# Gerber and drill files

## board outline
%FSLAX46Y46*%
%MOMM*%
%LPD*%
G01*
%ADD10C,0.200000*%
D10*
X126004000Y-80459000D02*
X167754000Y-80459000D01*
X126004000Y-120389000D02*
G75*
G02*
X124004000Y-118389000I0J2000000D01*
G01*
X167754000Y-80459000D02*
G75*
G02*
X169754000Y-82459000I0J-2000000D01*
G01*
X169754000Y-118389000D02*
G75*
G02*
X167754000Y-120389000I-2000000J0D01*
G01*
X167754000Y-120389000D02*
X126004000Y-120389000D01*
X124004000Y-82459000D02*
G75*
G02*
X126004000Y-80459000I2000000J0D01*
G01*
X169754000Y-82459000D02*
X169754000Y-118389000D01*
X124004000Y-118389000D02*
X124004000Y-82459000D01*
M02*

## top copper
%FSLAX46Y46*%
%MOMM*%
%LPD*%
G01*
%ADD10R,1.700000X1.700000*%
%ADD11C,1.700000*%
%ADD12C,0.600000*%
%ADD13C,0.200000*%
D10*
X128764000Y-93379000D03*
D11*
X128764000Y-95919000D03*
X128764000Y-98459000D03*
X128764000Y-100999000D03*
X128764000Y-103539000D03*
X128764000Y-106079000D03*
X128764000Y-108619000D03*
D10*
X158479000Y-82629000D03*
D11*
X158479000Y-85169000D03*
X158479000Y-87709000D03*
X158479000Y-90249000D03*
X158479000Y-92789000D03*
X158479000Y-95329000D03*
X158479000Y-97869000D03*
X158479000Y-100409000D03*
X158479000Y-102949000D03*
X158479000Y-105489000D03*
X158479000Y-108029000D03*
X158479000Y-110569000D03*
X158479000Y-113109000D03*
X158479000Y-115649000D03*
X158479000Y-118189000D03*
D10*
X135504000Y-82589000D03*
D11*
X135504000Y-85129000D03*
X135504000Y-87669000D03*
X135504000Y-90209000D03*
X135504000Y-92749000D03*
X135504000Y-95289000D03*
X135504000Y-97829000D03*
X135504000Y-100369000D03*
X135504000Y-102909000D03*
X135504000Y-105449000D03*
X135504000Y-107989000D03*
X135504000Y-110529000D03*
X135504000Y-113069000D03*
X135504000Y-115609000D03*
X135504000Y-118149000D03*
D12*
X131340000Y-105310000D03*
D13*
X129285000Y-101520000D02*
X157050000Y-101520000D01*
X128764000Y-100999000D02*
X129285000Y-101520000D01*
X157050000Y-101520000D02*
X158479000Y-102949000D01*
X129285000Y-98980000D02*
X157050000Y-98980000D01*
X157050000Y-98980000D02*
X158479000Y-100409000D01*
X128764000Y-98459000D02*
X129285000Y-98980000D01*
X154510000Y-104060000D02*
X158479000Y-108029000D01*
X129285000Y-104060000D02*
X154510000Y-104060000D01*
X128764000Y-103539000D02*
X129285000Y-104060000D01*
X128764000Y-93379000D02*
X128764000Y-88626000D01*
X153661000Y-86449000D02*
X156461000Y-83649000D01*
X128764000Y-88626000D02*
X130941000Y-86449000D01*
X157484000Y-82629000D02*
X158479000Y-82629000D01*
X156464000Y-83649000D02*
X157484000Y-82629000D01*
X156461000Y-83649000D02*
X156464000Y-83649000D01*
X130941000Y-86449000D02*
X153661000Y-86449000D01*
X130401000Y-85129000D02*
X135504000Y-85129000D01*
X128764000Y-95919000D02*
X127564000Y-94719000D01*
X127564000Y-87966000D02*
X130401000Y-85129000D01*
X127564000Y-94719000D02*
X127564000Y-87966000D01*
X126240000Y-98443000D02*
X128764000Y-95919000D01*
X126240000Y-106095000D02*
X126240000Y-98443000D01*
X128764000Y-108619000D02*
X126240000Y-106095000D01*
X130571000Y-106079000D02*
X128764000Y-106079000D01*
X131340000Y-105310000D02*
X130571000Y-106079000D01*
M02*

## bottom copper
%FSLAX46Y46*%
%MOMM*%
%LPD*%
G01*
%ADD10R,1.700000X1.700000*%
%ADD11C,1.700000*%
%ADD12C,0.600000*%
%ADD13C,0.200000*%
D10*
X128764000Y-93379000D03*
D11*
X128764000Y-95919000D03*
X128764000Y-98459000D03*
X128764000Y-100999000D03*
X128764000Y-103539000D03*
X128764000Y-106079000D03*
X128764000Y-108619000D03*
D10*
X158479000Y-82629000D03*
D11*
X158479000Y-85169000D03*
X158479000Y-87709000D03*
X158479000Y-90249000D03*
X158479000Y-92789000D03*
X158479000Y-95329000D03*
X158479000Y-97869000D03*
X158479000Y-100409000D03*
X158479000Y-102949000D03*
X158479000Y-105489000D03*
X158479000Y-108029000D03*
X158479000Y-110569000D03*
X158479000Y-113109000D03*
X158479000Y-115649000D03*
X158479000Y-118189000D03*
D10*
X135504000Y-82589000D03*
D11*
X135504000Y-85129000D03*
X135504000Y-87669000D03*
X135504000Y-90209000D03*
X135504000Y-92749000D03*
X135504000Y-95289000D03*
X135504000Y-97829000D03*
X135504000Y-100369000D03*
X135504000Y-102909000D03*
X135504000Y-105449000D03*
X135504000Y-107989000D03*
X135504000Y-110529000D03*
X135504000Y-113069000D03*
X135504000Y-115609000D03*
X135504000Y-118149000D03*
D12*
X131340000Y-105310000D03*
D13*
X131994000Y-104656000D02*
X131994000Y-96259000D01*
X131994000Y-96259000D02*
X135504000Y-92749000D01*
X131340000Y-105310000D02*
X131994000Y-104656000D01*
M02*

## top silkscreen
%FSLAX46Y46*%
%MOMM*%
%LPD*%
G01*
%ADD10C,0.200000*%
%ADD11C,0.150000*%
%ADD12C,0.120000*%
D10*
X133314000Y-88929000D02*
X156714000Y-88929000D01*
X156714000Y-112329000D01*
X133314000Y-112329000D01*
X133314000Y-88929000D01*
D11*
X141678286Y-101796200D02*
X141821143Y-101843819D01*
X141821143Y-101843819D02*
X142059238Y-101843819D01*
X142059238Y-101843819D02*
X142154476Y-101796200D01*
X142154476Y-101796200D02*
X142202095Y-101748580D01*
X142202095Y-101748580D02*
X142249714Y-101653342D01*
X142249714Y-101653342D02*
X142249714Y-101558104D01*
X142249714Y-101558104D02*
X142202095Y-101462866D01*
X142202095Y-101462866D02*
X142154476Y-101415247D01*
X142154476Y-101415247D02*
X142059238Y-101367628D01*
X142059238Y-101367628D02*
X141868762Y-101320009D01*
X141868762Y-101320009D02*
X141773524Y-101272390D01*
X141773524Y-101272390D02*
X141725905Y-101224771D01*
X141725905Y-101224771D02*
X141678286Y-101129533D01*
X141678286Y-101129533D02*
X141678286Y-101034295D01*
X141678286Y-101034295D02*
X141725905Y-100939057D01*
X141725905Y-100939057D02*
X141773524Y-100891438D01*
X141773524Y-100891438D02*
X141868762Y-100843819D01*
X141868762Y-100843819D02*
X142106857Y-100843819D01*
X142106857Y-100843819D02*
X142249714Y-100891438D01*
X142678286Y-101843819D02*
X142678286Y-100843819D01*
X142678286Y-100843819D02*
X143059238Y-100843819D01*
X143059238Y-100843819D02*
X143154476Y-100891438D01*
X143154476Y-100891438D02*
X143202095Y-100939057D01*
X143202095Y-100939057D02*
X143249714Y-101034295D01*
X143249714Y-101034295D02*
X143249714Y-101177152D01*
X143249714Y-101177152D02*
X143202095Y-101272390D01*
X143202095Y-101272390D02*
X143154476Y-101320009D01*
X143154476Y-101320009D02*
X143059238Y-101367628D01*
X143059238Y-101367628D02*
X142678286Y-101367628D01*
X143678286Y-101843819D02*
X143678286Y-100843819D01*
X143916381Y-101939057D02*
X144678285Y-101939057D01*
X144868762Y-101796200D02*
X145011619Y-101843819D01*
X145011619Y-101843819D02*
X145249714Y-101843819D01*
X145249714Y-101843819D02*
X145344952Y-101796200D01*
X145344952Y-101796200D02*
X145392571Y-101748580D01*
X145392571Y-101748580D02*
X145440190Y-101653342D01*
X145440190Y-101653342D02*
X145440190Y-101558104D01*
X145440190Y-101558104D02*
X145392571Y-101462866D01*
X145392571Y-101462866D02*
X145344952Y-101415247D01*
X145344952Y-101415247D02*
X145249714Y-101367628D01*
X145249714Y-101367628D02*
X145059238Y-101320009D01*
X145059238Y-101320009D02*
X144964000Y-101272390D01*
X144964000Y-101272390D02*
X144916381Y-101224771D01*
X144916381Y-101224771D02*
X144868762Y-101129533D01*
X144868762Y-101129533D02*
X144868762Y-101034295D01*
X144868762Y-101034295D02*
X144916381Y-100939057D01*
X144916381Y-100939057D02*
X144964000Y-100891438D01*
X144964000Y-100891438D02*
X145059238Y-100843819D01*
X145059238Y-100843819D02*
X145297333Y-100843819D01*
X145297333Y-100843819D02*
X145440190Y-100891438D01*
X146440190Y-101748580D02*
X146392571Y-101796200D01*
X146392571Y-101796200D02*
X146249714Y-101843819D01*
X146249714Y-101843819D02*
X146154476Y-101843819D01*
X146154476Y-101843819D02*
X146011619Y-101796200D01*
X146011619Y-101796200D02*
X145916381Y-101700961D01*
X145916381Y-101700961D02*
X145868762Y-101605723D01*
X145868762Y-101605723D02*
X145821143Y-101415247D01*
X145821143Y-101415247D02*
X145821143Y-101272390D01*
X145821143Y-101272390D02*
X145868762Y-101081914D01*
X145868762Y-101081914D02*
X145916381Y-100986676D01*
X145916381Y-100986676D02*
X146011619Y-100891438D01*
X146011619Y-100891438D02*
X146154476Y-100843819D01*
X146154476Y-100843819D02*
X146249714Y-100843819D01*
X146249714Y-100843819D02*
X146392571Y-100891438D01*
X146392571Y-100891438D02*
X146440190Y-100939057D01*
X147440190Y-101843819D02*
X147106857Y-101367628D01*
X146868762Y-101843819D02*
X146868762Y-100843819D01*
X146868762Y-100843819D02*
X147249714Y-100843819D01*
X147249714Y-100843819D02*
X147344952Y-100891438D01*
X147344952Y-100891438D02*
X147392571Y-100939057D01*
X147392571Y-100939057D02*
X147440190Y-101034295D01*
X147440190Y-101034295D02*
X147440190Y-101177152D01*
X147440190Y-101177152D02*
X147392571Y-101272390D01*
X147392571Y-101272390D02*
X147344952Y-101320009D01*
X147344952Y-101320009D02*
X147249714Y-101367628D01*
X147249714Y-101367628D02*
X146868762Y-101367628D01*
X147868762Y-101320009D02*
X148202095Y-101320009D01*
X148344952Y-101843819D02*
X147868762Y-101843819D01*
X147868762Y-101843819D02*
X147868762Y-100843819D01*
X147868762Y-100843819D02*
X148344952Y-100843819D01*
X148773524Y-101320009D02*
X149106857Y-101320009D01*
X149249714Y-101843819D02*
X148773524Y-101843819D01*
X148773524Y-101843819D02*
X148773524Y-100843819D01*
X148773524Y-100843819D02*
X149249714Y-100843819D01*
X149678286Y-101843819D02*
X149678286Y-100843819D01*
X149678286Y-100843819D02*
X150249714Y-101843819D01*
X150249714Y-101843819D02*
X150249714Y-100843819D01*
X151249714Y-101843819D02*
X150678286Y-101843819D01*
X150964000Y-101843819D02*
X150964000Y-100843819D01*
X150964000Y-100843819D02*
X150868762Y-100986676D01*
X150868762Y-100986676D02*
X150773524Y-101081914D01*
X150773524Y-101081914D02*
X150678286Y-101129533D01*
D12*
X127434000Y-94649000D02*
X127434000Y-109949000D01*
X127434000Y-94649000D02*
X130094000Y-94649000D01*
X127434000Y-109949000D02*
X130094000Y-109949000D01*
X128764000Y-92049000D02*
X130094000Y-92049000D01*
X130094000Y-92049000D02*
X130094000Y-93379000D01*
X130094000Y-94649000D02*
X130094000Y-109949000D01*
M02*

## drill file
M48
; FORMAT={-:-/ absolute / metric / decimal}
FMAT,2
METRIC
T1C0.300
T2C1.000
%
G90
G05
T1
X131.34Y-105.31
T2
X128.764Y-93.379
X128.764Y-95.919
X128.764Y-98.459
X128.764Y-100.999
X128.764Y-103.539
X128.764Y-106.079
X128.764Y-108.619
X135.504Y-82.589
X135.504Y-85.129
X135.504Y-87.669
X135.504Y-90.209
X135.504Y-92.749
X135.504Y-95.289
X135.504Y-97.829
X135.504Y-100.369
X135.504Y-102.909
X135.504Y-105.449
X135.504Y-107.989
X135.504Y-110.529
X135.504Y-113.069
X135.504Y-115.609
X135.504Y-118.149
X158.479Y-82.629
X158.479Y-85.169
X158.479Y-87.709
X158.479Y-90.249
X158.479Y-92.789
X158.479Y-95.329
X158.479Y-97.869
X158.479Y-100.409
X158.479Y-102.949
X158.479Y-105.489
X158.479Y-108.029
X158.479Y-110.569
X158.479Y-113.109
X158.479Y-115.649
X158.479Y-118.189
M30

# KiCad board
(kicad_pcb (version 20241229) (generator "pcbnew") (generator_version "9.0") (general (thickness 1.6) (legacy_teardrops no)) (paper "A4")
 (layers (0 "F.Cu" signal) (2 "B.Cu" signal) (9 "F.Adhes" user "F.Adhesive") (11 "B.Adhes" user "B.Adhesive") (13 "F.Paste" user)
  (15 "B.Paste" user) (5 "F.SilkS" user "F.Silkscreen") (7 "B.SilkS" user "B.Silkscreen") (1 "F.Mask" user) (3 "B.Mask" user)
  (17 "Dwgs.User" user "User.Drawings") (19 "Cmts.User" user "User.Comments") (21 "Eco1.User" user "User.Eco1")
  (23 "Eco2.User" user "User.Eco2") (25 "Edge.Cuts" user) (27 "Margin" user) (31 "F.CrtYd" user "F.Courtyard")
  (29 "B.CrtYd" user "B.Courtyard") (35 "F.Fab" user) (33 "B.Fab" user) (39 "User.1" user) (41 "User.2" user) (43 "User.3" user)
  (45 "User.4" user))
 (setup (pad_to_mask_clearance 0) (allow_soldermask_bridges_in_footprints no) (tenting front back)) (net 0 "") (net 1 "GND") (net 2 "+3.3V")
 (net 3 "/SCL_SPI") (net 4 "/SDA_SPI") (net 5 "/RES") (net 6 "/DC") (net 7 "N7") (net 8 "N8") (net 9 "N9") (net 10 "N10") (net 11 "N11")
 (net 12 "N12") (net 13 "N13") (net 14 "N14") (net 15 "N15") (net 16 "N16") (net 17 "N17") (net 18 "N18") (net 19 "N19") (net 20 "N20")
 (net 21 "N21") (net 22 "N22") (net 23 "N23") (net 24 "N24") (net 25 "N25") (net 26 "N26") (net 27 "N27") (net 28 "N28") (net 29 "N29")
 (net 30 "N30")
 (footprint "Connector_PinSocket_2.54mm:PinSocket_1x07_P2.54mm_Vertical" (layer "F.Cu") (at 128.764 93.379)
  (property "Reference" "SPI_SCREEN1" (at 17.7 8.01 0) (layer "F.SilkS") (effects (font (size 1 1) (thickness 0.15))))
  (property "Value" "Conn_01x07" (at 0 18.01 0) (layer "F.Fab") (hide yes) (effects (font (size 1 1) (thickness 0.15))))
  (fp_line (start -1.33 1.27) (end -1.33 16.57) (stroke (width 0.12) (type solid)) (layer "F.SilkS"))
  (fp_line (start -1.33 1.27) (end 1.33 1.27) (stroke (width 0.12) (type solid)) (layer "F.SilkS"))
  (fp_line (start -1.33 16.57) (end 1.33 16.57) (stroke (width 0.12) (type solid)) (layer "F.SilkS"))
  (fp_line (start 0 -1.33) (end 1.33 -1.33) (stroke (width 0.12) (type solid)) (layer "F.SilkS"))
  (fp_line (start 1.33 -1.33) (end 1.33 0) (stroke (width 0.12) (type solid)) (layer "F.SilkS"))
  (fp_line (start 1.33 1.27) (end 1.33 16.57) (stroke (width 0.12) (type solid)) (layer "F.SilkS"))
  (pad "1" thru_hole rect (at 0 0) (size 1.7 1.7) (drill 1) (layers "*.Cu" "*.Mask") (remove_unused_layers no) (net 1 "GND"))
  (pad "2" thru_hole circle (at 0 2.54) (size 1.7 1.7) (drill 1) (layers "*.Cu" "*.Mask") (remove_unused_layers no) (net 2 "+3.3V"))
  (pad "3" thru_hole circle (at 0 5.08) (size 1.7 1.7) (drill 1) (layers "*.Cu" "*.Mask") (remove_unused_layers no) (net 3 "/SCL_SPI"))
  (pad "4" thru_hole circle (at 0 7.62) (size 1.7 1.7) (drill 1) (layers "*.Cu" "*.Mask") (remove_unused_layers no) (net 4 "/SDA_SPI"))
  (pad "5" thru_hole circle (at 0 10.16) (size 1.7 1.7) (drill 1) (layers "*.Cu" "*.Mask") (remove_unused_layers no) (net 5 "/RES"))
  (pad "6" thru_hole circle (at 0 12.7) (size 1.7 1.7) (drill 1) (layers "*.Cu" "*.Mask") (remove_unused_layers no) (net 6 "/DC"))
  (pad "7" thru_hole circle (at 0 15.24) (size 1.7 1.7) (drill 1) (layers "*.Cu" "*.Mask") (remove_unused_layers no) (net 2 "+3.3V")))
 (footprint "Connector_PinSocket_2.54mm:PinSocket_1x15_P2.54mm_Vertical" (layer "B.Cu") (at 158.479 82.629 180)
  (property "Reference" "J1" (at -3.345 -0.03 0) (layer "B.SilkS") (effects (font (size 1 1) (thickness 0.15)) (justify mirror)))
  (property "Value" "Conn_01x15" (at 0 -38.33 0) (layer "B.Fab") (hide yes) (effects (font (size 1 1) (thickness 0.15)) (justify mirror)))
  (pad "1" thru_hole rect (at 0 0 180) (size 1.7 1.7) (drill 1) (layers "*.Cu" "*.Mask") (remove_unused_layers no) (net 1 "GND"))
  (pad "2" thru_hole circle (at 0 -2.54 180) (size 1.7 1.7) (drill 1) (layers "*.Cu" "*.Mask") (remove_unused_layers no) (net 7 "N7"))
  (pad "3" thru_hole circle (at 0 -5.08 180) (size 1.7 1.7) (drill 1) (layers "*.Cu" "*.Mask") (remove_unused_layers no) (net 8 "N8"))
  (pad "4" thru_hole circle (at 0 -7.62 180) (size 1.7 1.7) (drill 1) (layers "*.Cu" "*.Mask") (remove_unused_layers no) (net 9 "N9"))
  (pad "5" thru_hole circle (at 0 -10.16 180) (size 1.7 1.7) (drill 1) (layers "*.Cu" "*.Mask") (remove_unused_layers no) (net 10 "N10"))
  (pad "6" thru_hole circle (at 0 -12.7 180) (size 1.7 1.7) (drill 1) (layers "*.Cu" "*.Mask") (remove_unused_layers no) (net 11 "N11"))
  (pad "7" thru_hole circle (at 0 -15.24 180) (size 1.7 1.7) (drill 1) (layers "*.Cu" "*.Mask") (remove_unused_layers no) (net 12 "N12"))
  (pad "8" thru_hole circle (at 0 -17.78 180) (size 1.7 1.7) (drill 1) (layers "*.Cu" "*.Mask") (remove_unused_layers no) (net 3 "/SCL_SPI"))
  (pad "9" thru_hole circle (at 0 -20.32 180) (size 1.7 1.7) (drill 1) (layers "*.Cu" "*.Mask") (remove_unused_layers no) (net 4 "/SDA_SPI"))
  (pad "10" thru_hole circle (at 0 -22.86 180) (size 1.7 1.7) (drill 1) (layers "*.Cu" "*.Mask") (remove_unused_layers no) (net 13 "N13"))
  (pad "11" thru_hole circle (at 0 -25.4 180) (size 1.7 1.7) (drill 1) (layers "*.Cu" "*.Mask") (remove_unused_layers no) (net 5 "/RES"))
  (pad "12" thru_hole circle (at 0 -27.94 180) (size 1.7 1.7) (drill 1) (layers "*.Cu" "*.Mask") (remove_unused_layers no) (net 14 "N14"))
  (pad "13" thru_hole circle (at 0 -30.48 180) (size 1.7 1.7) (drill 1) (layers "*.Cu" "*.Mask") (remove_unused_layers no) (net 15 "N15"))
  (pad "14" thru_hole circle (at 0 -33.02 180) (size 1.7 1.7) (drill 1) (layers "*.Cu" "*.Mask") (remove_unused_layers no) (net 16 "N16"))
  (pad "15" thru_hole circle (at 0 -35.56 180) (size 1.7 1.7) (drill 1) (layers "*.Cu" "*.Mask") (remove_unused_layers no) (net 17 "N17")))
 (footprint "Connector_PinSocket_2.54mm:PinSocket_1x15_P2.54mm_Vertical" (layer "B.Cu") (at 135.504 82.589 180)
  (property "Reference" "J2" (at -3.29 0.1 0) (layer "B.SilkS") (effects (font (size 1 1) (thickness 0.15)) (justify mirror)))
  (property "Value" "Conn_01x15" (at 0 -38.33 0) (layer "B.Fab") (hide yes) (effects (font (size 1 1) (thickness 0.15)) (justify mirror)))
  (pad "1" thru_hole rect (at 0 0 180) (size 1.7 1.7) (drill 1) (layers "*.Cu" "*.Mask") (remove_unused_layers no) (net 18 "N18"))
  (pad "2" thru_hole circle (at 0 -2.54 180) (size 1.7 1.7) (drill 1) (layers "*.Cu" "*.Mask") (remove_unused_layers no) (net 2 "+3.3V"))
  (pad "3" thru_hole circle (at 0 -5.08 180) (size 1.7 1.7) (drill 1) (layers "*.Cu" "*.Mask") (remove_unused_layers no) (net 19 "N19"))
  (pad "4" thru_hole circle (at 0 -7.62 180) (size 1.7 1.7) (drill 1) (layers "*.Cu" "*.Mask") (remove_unused_layers no) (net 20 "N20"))
  (pad "5" thru_hole circle (at 0 -10.16 180) (size 1.7 1.7) (drill 1) (layers "*.Cu" "*.Mask") (remove_unused_layers no) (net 6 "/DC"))
  (pad "6" thru_hole circle (at 0 -12.7 180) (size 1.7 1.7) (drill 1) (layers "*.Cu" "*.Mask") (remove_unused_layers no) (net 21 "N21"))
  (pad "7" thru_hole circle (at 0 -15.24 180) (size 1.7 1.7) (drill 1) (layers "*.Cu" "*.Mask") (remove_unused_layers no) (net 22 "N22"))
  (pad "8" thru_hole circle (at 0 -17.78 180) (size 1.7 1.7) (drill 1) (layers "*.Cu" "*.Mask") (remove_unused_layers no) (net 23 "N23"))
  (pad "9" thru_hole circle (at 0 -20.32 180) (size 1.7 1.7) (drill 1) (layers "*.Cu" "*.Mask") (remove_unused_layers no) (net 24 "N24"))
  (pad "10" thru_hole circle (at 0 -22.86 180) (size 1.7 1.7) (drill 1) (layers "*.Cu" "*.Mask") (remove_unused_layers no) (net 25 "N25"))
  (pad "11" thru_hole circle (at 0 -25.4 180) (size 1.7 1.7) (drill 1) (layers "*.Cu" "*.Mask") (remove_unused_layers no) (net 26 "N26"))
  (pad "12" thru_hole circle (at 0 -27.94 180) (size 1.7 1.7) (drill 1) (layers "*.Cu" "*.Mask") (remove_unused_layers no) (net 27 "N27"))
  (pad "13" thru_hole circle (at 0 -30.48 180) (size 1.7 1.7) (drill 1) (layers "*.Cu" "*.Mask") (remove_unused_layers no) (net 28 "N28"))
  (pad "14" thru_hole circle (at 0 -33.02 180) (size 1.7 1.7) (drill 1) (layers "*.Cu" "*.Mask") (remove_unused_layers no) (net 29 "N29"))
  (pad "15" thru_hole circle (at 0 -35.56 180) (size 1.7 1.7) (drill 1) (layers "*.Cu" "*.Mask") (remove_unused_layers no) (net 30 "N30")))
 (gr_rect (start 133.314 88.929) (end 156.714 112.329) (stroke (width 0.2) (type solid)) (fill no) (layer "F.SilkS"))
 (gr_line (start 126.004 80.459) (end 167.754 80.459) (stroke (width 0.2) (type default)) (layer "Edge.Cuts"))
 (gr_arc (start 126.004 120.389) (mid 124.589786 119.803214) (end 124.004 118.389) (stroke (width 0.2) (type default)) (layer "Edge.Cuts"))
 (gr_arc (start 167.754 80.459) (mid 169.168214 81.044786) (end 169.754 82.459) (stroke (width 0.2) (type default)) (layer "Edge.Cuts"))
 (gr_arc (start 169.754 118.389) (mid 169.168214 119.803214) (end 167.754 120.389) (stroke (width 0.2) (type default)) (layer "Edge.Cuts"))
 (gr_line (start 167.754 120.389) (end 126.004 120.389) (stroke (width 0.2) (type default)) (layer "Edge.Cuts"))
 (gr_arc (start 124.004 82.459) (mid 124.589786 81.044786) (end 126.004 80.459) (stroke (width 0.2) (type default)) (layer "Edge.Cuts"))
 (gr_line (start 169.754 82.459) (end 169.754 118.389) (stroke (width 0.2) (type default)) (layer "Edge.Cuts"))
 (gr_line (start 124.004 118.389) (end 124.004 82.459) (stroke (width 0.2) (type default)) (layer "Edge.Cuts"))
 (segment (start 129.285 101.52) (end 157.05 101.52) (width 0.2) (layer "F.Cu") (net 4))
 (segment (start 128.764 100.999) (end 129.285 101.52) (width 0.2) (layer "F.Cu") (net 4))
 (segment (start 157.05 101.52) (end 158.479 102.949) (width 0.2) (layer "F.Cu") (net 4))
 (segment (start 129.285 98.98) (end 157.05 98.98) (width 0.2) (layer "F.Cu") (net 3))
 (segment (start 157.05 98.98) (end 158.479 100.409) (width 0.2) (layer "F.Cu") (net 3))
 (segment (start 128.764 98.459) (end 129.285 98.98) (width 0.2) (layer "F.Cu") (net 3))
 (segment (start 154.51 104.06) (end 158.479 108.029) (width 0.2) (layer "F.Cu") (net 5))
 (segment (start 129.285 104.06) (end 154.51 104.06) (width 0.2) (layer "F.Cu") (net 5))
 (segment (start 128.764 103.539) (end 129.285 104.06) (width 0.2) (layer "F.Cu") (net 5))
 (segment (start 128.764 93.379) (end 128.764 88.626) (width 0.2) (layer "F.Cu") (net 1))
 (segment (start 153.661 86.449) (end 156.461 83.649) (width 0.2) (layer "F.Cu") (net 1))
 (segment (start 128.764 88.626) (end 130.941 86.449) (width 0.2) (layer "F.Cu") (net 1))
 (segment (start 157.484 82.629) (end 158.479 82.629) (width 0.2) (layer "F.Cu") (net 1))
 (segment (start 156.464 83.649) (end 157.484 82.629) (width 0.2) (layer "F.Cu") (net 1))
 (segment (start 156.461 83.649) (end 156.464 83.649) (width 0.2) (layer "F.Cu") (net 1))
 (segment (start 130.941 86.449) (end 153.661 86.449) (width 0.2) (layer "F.Cu") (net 1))
 (segment (start 130.401 85.129) (end 135.504 85.129) (width 0.2) (layer "F.Cu") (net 2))
 (segment (start 128.764 95.919) (end 127.564 94.719) (width 0.2) (layer "F.Cu") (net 2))
 (segment (start 127.564 87.966) (end 130.401 85.129) (width 0.2) (layer "F.Cu") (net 2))
 (segment (start 127.564 94.719) (end 127.564 87.966) (width 0.2) (layer "F.Cu") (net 2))
 (segment (start 126.24 98.443) (end 128.764 95.919) (width 0.2) (layer "F.Cu") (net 2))
 (segment (start 126.24 106.095) (end 126.24 98.443) (width 0.2) (layer "F.Cu") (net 2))
 (segment (start 128.764 108.619) (end 126.24 106.095) (width 0.2) (layer "F.Cu") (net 2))
 (segment (start 130.571 106.079) (end 128.764 106.079) (width 0.2) (layer "F.Cu") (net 6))
 (segment (start 131.34 105.31) (end 130.571 106.079) (width 0.2) (layer "F.Cu") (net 6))
 (via (at 131.34 105.31) (size 0.6) (drill 0.3) (layers "F.Cu" "B.Cu") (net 6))
 (segment (start 131.994 104.656) (end 131.994 96.259) (width 0.2) (layer "B.Cu") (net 6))
 (segment (start 131.994 96.259) (end 135.504 92.749) (width 0.2) (layer "B.Cu") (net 6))
 (segment (start 131.34 105.31) (end 131.994 104.656) (width 0.2) (layer "B.Cu") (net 6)))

